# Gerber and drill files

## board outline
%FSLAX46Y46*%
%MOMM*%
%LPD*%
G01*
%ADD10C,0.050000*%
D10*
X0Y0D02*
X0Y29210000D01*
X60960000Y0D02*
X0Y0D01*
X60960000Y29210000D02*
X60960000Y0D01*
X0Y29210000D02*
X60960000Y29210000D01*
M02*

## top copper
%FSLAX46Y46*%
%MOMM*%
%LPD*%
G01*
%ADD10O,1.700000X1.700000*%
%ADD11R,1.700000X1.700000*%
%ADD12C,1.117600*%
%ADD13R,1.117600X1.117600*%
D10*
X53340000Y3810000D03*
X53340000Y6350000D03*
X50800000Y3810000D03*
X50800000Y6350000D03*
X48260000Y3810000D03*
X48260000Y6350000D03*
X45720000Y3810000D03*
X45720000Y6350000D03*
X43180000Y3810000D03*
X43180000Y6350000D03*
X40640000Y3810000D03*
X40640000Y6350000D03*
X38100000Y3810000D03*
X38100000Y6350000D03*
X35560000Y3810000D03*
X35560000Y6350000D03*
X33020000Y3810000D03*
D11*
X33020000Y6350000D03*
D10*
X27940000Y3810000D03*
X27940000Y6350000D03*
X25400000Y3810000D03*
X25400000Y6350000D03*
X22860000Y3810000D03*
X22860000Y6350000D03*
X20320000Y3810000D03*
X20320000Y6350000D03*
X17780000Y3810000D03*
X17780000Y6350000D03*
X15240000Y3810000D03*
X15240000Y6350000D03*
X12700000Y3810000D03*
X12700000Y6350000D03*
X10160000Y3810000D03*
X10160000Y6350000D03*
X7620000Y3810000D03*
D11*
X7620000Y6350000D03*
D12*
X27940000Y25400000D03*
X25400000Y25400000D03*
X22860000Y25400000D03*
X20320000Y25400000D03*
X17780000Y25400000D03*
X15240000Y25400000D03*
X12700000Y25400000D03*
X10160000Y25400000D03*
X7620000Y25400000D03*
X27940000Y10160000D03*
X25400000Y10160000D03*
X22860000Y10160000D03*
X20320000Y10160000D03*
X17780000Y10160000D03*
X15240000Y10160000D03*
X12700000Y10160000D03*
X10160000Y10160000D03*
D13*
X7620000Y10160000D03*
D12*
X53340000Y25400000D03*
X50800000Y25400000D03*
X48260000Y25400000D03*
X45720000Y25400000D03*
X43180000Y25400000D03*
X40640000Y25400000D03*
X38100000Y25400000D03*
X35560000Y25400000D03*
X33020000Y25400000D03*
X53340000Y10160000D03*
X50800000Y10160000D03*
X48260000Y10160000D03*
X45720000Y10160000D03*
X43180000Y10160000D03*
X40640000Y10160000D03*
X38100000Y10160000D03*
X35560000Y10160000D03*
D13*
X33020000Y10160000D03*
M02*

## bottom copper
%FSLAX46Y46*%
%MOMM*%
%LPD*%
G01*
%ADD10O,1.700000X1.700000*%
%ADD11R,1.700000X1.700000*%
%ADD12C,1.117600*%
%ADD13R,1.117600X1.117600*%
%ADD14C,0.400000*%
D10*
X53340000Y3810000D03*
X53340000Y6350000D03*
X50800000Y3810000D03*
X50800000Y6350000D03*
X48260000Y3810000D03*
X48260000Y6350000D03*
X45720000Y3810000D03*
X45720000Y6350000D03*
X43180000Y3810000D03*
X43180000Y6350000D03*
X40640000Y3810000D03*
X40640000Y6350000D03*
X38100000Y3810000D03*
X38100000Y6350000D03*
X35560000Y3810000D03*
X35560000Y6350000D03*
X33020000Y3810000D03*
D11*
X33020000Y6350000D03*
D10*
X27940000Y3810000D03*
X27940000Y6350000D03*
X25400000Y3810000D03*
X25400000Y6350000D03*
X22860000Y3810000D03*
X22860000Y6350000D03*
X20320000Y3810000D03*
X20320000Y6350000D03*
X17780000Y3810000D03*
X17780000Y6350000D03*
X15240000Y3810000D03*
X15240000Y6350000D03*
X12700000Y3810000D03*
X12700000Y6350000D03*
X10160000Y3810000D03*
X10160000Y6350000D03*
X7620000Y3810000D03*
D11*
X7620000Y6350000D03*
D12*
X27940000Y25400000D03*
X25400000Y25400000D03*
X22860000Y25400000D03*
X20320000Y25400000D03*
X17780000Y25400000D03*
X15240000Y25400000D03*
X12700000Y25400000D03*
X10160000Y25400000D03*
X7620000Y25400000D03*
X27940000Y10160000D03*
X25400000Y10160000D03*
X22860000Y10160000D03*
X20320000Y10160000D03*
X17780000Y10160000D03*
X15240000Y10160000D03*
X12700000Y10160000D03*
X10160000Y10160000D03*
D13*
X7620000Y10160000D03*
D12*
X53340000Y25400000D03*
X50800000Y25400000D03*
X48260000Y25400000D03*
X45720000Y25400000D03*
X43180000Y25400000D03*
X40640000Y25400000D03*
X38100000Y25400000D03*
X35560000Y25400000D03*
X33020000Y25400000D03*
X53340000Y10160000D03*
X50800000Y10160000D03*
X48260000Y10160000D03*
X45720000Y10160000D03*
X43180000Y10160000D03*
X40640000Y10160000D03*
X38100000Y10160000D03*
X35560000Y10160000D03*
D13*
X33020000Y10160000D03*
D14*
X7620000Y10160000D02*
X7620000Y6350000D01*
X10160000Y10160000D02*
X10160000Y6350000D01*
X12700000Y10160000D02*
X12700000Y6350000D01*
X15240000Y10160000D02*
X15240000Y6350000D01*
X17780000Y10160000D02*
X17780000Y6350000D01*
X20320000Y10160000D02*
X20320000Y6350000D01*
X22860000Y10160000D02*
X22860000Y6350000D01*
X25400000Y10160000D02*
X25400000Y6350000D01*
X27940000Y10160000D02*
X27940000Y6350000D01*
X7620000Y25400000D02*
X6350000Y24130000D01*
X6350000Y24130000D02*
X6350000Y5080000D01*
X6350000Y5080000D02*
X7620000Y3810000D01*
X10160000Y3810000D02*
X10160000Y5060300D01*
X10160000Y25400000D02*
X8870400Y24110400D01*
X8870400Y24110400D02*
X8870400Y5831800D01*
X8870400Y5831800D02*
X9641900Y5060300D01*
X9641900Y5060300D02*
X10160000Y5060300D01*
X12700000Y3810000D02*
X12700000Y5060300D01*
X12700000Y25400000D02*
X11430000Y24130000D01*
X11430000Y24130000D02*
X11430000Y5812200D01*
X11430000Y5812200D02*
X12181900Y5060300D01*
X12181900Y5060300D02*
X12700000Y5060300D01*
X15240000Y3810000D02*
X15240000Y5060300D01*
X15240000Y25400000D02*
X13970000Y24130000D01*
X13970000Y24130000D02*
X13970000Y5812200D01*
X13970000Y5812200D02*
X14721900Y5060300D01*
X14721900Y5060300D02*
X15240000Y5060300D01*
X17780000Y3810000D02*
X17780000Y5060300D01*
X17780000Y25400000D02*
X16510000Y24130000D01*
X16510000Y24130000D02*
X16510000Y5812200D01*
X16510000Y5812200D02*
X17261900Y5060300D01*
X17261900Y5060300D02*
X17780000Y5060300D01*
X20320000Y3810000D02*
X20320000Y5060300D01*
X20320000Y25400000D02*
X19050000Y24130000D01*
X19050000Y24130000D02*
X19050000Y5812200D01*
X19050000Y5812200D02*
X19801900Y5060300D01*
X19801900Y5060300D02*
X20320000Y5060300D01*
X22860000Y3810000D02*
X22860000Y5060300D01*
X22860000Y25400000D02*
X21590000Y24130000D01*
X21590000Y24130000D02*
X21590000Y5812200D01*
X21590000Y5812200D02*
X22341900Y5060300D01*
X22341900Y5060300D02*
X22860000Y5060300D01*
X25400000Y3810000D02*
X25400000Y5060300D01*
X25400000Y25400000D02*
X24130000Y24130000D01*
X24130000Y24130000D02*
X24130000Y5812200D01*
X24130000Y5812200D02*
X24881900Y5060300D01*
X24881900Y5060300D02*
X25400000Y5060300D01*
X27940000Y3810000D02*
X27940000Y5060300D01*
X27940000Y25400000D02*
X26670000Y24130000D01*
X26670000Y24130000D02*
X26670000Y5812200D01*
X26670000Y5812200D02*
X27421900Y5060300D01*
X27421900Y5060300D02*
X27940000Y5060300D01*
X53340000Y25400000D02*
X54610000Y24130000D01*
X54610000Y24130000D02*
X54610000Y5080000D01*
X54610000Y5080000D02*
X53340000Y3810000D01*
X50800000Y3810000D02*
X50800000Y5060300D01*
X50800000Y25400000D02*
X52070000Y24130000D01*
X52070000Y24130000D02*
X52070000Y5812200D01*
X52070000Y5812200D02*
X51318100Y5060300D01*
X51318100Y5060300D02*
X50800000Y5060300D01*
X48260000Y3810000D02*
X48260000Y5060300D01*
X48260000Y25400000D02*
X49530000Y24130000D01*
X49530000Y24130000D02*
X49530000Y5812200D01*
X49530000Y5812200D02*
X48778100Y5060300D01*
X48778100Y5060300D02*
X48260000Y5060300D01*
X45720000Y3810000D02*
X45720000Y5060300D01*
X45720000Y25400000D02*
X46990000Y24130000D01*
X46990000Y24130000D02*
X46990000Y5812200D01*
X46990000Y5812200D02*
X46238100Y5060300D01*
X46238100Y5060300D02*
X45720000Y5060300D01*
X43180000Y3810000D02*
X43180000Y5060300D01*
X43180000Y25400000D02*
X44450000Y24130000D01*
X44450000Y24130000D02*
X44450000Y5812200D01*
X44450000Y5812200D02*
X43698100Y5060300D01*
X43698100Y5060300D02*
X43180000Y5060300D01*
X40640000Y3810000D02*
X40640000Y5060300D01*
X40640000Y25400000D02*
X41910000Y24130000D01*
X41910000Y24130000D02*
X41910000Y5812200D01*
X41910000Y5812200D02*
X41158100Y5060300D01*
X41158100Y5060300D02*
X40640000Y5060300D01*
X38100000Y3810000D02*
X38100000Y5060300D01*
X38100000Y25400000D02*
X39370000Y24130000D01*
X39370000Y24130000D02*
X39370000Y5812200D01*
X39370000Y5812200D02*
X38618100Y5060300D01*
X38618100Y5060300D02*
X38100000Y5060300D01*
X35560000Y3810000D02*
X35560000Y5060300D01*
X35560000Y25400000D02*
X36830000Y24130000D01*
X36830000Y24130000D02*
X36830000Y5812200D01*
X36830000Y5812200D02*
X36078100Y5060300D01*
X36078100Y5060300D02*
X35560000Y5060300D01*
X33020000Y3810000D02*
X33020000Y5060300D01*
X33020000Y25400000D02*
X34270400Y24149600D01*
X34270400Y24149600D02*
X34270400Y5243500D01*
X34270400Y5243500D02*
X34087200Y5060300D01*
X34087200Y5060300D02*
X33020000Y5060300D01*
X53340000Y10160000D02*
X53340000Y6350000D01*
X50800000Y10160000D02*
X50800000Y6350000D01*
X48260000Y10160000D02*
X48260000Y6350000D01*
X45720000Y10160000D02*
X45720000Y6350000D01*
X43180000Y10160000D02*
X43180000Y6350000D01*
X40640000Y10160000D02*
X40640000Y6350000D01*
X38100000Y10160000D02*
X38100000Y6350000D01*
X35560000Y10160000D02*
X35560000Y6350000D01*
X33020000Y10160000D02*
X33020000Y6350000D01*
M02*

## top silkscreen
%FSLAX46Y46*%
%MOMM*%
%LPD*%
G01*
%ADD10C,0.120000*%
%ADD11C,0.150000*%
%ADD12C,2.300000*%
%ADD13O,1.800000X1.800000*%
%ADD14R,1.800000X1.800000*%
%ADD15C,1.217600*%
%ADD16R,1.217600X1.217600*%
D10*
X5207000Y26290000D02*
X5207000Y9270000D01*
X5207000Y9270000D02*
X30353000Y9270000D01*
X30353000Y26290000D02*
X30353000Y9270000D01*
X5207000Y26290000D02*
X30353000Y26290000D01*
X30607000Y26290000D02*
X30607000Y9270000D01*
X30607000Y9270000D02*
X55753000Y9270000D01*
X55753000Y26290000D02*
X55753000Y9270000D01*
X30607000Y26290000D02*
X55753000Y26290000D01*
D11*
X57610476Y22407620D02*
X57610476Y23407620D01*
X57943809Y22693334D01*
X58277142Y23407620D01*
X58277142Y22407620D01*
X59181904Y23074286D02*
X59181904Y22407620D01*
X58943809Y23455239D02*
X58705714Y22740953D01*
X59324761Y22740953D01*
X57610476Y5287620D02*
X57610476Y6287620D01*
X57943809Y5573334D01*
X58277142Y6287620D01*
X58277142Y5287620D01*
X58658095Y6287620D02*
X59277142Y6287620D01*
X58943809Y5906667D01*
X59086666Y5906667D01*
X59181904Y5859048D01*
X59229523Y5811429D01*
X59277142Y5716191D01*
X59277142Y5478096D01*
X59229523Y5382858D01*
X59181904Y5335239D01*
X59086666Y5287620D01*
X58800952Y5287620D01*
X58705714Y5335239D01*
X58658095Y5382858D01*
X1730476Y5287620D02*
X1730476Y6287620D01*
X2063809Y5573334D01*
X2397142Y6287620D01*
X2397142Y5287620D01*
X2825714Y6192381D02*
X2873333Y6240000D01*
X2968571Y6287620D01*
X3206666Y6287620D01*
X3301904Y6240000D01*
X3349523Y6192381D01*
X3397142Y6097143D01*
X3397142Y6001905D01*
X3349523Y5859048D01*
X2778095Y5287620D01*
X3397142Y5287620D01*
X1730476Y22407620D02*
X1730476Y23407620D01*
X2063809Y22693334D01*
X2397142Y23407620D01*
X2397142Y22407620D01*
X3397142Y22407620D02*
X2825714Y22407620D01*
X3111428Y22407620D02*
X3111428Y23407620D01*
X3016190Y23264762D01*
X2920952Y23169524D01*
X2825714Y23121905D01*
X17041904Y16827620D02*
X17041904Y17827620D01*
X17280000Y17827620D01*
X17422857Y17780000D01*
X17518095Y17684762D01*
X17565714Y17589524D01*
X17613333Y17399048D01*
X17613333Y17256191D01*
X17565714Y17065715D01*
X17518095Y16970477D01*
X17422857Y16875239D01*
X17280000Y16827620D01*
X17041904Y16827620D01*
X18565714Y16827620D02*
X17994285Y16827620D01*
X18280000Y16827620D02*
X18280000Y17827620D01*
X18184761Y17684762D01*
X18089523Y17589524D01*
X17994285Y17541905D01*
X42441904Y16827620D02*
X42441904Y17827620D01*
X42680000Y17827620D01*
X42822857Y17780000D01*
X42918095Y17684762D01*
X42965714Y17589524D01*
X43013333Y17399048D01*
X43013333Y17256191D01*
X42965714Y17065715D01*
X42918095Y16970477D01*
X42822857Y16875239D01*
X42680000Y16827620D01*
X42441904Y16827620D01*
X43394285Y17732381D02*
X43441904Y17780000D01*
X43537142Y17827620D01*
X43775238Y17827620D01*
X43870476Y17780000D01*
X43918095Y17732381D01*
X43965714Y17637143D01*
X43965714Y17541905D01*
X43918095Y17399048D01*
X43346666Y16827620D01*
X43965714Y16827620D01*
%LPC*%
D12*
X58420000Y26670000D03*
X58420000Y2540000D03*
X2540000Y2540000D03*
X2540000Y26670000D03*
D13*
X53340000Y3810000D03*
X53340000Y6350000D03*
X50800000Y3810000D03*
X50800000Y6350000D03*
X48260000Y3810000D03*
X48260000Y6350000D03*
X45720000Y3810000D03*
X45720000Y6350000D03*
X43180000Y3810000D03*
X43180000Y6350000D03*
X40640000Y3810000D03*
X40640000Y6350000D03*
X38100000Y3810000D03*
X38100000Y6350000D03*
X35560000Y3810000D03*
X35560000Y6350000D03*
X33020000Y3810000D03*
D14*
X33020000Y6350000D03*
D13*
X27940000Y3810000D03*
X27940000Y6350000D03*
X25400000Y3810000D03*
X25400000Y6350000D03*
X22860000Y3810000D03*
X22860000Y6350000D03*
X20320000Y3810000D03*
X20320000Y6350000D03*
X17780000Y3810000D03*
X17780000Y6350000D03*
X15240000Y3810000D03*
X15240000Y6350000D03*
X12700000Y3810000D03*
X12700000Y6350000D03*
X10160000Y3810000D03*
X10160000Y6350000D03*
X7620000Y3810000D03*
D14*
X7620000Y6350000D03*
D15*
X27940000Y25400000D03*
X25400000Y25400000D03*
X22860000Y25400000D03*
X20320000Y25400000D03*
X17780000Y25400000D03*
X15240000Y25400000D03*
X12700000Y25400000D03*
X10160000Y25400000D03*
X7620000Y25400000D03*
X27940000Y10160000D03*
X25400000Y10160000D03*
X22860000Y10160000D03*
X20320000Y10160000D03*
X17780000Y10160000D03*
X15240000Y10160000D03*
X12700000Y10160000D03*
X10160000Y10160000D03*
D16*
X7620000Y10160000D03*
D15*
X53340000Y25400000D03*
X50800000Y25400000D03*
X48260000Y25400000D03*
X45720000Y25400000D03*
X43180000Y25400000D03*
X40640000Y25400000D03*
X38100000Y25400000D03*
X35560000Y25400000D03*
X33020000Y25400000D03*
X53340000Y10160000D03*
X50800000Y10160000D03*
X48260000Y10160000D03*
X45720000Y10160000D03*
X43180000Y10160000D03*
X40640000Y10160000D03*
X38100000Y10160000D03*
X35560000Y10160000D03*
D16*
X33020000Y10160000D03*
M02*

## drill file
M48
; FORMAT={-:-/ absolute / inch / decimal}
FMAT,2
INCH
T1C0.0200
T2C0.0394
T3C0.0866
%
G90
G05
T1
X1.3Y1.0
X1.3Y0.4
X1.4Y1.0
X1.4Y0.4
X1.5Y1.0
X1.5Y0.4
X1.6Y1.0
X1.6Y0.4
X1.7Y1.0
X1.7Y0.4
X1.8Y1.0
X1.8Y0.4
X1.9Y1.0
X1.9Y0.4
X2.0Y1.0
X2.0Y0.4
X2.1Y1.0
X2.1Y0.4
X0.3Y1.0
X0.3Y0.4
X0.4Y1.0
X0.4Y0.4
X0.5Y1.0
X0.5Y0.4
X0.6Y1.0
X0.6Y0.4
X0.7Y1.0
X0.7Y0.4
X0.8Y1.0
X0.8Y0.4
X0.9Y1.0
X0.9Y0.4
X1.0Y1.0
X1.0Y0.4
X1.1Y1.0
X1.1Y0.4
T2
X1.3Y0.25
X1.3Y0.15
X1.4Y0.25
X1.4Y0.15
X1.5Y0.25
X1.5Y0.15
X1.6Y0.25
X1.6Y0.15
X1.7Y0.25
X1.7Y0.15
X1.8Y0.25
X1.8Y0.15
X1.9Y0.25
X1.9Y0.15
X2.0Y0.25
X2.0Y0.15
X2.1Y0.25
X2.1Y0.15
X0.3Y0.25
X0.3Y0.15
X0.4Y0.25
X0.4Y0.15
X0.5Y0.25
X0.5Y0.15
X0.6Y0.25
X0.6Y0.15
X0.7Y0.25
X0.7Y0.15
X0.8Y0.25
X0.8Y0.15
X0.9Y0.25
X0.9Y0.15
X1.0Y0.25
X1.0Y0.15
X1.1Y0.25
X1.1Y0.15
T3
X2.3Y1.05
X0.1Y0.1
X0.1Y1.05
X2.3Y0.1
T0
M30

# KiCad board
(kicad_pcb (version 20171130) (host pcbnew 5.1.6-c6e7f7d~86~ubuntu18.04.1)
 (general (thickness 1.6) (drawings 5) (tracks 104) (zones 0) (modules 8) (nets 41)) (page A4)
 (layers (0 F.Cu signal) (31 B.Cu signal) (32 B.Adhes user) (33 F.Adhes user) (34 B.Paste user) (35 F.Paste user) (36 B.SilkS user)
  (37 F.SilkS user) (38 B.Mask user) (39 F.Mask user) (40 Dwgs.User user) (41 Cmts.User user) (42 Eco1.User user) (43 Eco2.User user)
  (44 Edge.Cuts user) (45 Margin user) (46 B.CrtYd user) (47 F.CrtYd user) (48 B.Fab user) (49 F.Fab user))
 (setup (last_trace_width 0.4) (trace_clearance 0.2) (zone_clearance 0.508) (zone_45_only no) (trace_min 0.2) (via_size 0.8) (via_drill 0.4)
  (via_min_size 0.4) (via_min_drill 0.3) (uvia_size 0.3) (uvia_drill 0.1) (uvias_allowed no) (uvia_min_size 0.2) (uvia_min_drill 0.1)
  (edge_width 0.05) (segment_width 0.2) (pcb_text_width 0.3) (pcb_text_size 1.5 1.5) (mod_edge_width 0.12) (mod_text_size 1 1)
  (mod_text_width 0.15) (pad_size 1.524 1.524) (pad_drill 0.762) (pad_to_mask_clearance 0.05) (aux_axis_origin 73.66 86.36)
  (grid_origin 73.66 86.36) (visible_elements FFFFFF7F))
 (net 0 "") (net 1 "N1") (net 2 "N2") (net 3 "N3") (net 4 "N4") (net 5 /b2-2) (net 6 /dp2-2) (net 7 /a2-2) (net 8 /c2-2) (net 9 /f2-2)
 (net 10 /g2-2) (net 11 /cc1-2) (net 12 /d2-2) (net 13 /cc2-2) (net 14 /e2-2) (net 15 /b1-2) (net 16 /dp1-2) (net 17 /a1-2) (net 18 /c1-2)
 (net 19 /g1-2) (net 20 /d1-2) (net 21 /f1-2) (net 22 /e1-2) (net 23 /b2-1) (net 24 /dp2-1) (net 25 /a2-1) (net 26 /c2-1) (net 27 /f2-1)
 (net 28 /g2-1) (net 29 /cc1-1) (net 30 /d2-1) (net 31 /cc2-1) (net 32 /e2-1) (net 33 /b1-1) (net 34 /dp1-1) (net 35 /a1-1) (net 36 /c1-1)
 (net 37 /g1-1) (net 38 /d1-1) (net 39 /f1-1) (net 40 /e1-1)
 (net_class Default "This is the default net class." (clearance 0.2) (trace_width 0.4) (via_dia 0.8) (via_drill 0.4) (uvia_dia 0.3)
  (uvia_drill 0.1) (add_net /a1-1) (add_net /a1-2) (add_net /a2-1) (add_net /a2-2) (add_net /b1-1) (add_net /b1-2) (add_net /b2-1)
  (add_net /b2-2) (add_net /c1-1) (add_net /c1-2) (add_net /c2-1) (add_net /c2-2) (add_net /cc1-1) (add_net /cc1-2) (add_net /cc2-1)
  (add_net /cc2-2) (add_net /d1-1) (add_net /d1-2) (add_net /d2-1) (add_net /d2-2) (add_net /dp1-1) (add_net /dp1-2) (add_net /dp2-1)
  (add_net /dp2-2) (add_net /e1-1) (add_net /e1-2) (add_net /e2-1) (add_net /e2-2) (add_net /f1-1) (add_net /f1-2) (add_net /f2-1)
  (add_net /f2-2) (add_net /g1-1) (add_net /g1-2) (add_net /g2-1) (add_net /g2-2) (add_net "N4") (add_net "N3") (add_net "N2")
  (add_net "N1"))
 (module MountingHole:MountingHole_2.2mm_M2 (layer F.Cu) (at 132.08 59.69)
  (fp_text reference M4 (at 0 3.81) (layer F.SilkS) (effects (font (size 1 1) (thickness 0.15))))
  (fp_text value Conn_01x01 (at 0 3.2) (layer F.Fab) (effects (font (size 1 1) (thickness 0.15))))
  (pad 1 np_thru_hole circle (at 0 0) (size 2.2 2.2) (drill 2.2) (layers *.Cu *.Mask) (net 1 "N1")))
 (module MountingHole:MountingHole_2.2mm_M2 (layer F.Cu) (at 132.08 83.82)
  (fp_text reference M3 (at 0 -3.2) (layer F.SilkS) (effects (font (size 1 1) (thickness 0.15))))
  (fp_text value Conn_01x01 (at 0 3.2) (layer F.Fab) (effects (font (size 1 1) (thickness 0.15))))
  (pad 1 np_thru_hole circle (at 0 0) (size 2.2 2.2) (drill 2.2) (layers *.Cu *.Mask) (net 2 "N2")))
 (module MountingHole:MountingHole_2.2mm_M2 (layer F.Cu) (at 76.2 83.82)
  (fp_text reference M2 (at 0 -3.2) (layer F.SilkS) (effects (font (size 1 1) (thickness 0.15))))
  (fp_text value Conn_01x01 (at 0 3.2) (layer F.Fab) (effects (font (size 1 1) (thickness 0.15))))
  (pad 1 np_thru_hole circle (at 0 0) (size 2.2 2.2) (drill 2.2) (layers *.Cu *.Mask) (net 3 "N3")))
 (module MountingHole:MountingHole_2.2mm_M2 (layer F.Cu) (at 76.2 59.69)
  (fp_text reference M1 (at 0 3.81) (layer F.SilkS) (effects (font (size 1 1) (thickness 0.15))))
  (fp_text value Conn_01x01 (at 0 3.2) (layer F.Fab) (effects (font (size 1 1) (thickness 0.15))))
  (pad 1 np_thru_hole circle (at 0 0) (size 2.2 2.2) (drill 2.2) (layers *.Cu *.Mask) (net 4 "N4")))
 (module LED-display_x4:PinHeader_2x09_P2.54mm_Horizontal (layer B.Cu) (at 106.68 80.01 270)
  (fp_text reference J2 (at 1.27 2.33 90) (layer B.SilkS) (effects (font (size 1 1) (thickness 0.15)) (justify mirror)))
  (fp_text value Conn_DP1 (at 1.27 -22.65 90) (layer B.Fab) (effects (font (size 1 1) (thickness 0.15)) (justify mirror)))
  (pad 10 thru_hole oval (at 2.54 -20.32 270) (size 1.7 1.7) (drill 1) (layers *.Cu *.Mask) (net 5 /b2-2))
  (pad 9 thru_hole oval (at 0 -20.32 270) (size 1.7 1.7) (drill 1) (layers *.Cu *.Mask) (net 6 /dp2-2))
  (pad 11 thru_hole oval (at 2.54 -17.78 270) (size 1.7 1.7) (drill 1) (layers *.Cu *.Mask) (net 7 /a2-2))
  (pad 8 thru_hole oval (at 0 -17.78 270) (size 1.7 1.7) (drill 1) (layers *.Cu *.Mask) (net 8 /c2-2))
  (pad 12 thru_hole oval (at 2.54 -15.24 270) (size 1.7 1.7) (drill 1) (layers *.Cu *.Mask) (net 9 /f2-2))
  (pad 7 thru_hole oval (at 0 -15.24 270) (size 1.7 1.7) (drill 1) (layers *.Cu *.Mask) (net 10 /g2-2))
  (pad 13 thru_hole oval (at 2.54 -12.7 270) (size 1.7 1.7) (drill 1) (layers *.Cu *.Mask) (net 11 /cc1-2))
  (pad 6 thru_hole oval (at 0 -12.7 270) (size 1.7 1.7) (drill 1) (layers *.Cu *.Mask) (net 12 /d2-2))
  (pad 14 thru_hole oval (at 2.54 -10.16 270) (size 1.7 1.7) (drill 1) (layers *.Cu *.Mask) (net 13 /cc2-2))
  (pad 5 thru_hole oval (at 0 -10.16 270) (size 1.7 1.7) (drill 1) (layers *.Cu *.Mask) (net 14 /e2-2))
  (pad 15 thru_hole oval (at 2.54 -7.62 270) (size 1.7 1.7) (drill 1) (layers *.Cu *.Mask) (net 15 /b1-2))
  (pad 4 thru_hole oval (at 0 -7.62 270) (size 1.7 1.7) (drill 1) (layers *.Cu *.Mask) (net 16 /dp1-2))
  (pad 16 thru_hole oval (at 2.54 -5.08 270) (size 1.7 1.7) (drill 1) (layers *.Cu *.Mask) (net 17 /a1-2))
  (pad 3 thru_hole oval (at 0 -5.08 270) (size 1.7 1.7) (drill 1) (layers *.Cu *.Mask) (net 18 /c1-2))
  (pad 17 thru_hole oval (at 2.54 -2.54 270) (size 1.7 1.7) (drill 1) (layers *.Cu *.Mask) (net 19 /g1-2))
  (pad 2 thru_hole oval (at 0 -2.54 270) (size 1.7 1.7) (drill 1) (layers *.Cu *.Mask) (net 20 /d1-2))
  (pad 18 thru_hole oval (at 2.54 0 270) (size 1.7 1.7) (drill 1) (layers *.Cu *.Mask) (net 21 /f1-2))
  (pad 1 thru_hole rect (at 0 0 270) (size 1.7 1.7) (drill 1) (layers *.Cu *.Mask) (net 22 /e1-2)))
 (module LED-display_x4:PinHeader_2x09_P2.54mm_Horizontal (layer B.Cu) (at 81.28 80.01 270)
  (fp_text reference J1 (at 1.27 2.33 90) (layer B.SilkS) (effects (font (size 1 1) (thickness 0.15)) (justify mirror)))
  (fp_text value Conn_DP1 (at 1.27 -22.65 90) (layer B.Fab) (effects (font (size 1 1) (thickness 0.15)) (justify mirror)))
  (pad 10 thru_hole oval (at 2.54 -20.32 270) (size 1.7 1.7) (drill 1) (layers *.Cu *.Mask) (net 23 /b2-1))
  (pad 9 thru_hole oval (at 0 -20.32 270) (size 1.7 1.7) (drill 1) (layers *.Cu *.Mask) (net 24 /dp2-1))
  (pad 11 thru_hole oval (at 2.54 -17.78 270) (size 1.7 1.7) (drill 1) (layers *.Cu *.Mask) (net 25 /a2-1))
  (pad 8 thru_hole oval (at 0 -17.78 270) (size 1.7 1.7) (drill 1) (layers *.Cu *.Mask) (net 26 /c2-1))
  (pad 12 thru_hole oval (at 2.54 -15.24 270) (size 1.7 1.7) (drill 1) (layers *.Cu *.Mask) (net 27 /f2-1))
  (pad 7 thru_hole oval (at 0 -15.24 270) (size 1.7 1.7) (drill 1) (layers *.Cu *.Mask) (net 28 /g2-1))
  (pad 13 thru_hole oval (at 2.54 -12.7 270) (size 1.7 1.7) (drill 1) (layers *.Cu *.Mask) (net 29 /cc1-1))
  (pad 6 thru_hole oval (at 0 -12.7 270) (size 1.7 1.7) (drill 1) (layers *.Cu *.Mask) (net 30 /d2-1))
  (pad 14 thru_hole oval (at 2.54 -10.16 270) (size 1.7 1.7) (drill 1) (layers *.Cu *.Mask) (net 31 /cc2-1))
  (pad 5 thru_hole oval (at 0 -10.16 270) (size 1.7 1.7) (drill 1) (layers *.Cu *.Mask) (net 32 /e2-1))
  (pad 15 thru_hole oval (at 2.54 -7.62 270) (size 1.7 1.7) (drill 1) (layers *.Cu *.Mask) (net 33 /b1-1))
  (pad 4 thru_hole oval (at 0 -7.62 270) (size 1.7 1.7) (drill 1) (layers *.Cu *.Mask) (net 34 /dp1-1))
  (pad 16 thru_hole oval (at 2.54 -5.08 270) (size 1.7 1.7) (drill 1) (layers *.Cu *.Mask) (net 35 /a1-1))
  (pad 3 thru_hole oval (at 0 -5.08 270) (size 1.7 1.7) (drill 1) (layers *.Cu *.Mask) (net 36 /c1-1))
  (pad 17 thru_hole oval (at 2.54 -2.54 270) (size 1.7 1.7) (drill 1) (layers *.Cu *.Mask) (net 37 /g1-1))
  (pad 2 thru_hole oval (at 0 -2.54 270) (size 1.7 1.7) (drill 1) (layers *.Cu *.Mask) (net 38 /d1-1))
  (pad 18 thru_hole oval (at 2.54 0 270) (size 1.7 1.7) (drill 1) (layers *.Cu *.Mask) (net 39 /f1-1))
  (pad 1 thru_hole rect (at 0 0 270) (size 1.7 1.7) (drill 1) (layers *.Cu *.Mask) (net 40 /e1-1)))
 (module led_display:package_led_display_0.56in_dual (layer F.Cu) (at 91.44 68.58)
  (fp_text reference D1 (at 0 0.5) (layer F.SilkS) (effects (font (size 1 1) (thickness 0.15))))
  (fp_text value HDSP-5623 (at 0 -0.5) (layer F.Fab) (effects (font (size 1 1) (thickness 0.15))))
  (fp_line (start -12.573 -8.51) (end -12.573 8.51) (layer F.SilkS) (width 0.12))
  (fp_line (start -12.573 8.51) (end 12.573 8.51) (layer F.SilkS) (width 0.12))
  (fp_line (start 12.573 -8.51) (end 12.573 8.51) (layer F.SilkS) (width 0.12))
  (fp_line (start -12.573 -8.51) (end 12.573 -8.51) (layer F.SilkS) (width 0.12))
  (pad 10 thru_hole circle (at 10.16 -7.62) (size 1.1176 1.1176) (drill 0.508) (layers *.Cu *.Mask) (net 23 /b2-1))
  (pad 11 thru_hole circle (at 7.62 -7.62) (size 1.1176 1.1176) (drill 0.508) (layers *.Cu *.Mask) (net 25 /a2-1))
  (pad 12 thru_hole circle (at 5.08 -7.62) (size 1.1176 1.1176) (drill 0.508) (layers *.Cu *.Mask) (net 27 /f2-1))
  (pad 13 thru_hole circle (at 2.54 -7.62) (size 1.1176 1.1176) (drill 0.508) (layers *.Cu *.Mask) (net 29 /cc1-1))
  (pad 14 thru_hole circle (at 0 -7.62) (size 1.1176 1.1176) (drill 0.508) (layers *.Cu *.Mask) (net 31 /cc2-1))
  (pad 15 thru_hole circle (at -2.54 -7.62) (size 1.1176 1.1176) (drill 0.508) (layers *.Cu *.Mask) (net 33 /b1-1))
  (pad 16 thru_hole circle (at -5.08 -7.62) (size 1.1176 1.1176) (drill 0.508) (layers *.Cu *.Mask) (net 35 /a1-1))
  (pad 17 thru_hole circle (at -7.62 -7.62) (size 1.1176 1.1176) (drill 0.508) (layers *.Cu *.Mask) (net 37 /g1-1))
  (pad 18 thru_hole circle (at -10.16 -7.62) (size 1.1176 1.1176) (drill 0.508) (layers *.Cu *.Mask) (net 39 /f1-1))
  (pad 9 thru_hole circle (at 10.16 7.62) (size 1.1176 1.1176) (drill 0.508) (layers *.Cu *.Mask) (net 24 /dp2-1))
  (pad 8 thru_hole circle (at 7.62 7.62) (size 1.1176 1.1176) (drill 0.508) (layers *.Cu *.Mask) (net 26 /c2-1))
  (pad 7 thru_hole circle (at 5.08 7.62) (size 1.1176 1.1176) (drill 0.508) (layers *.Cu *.Mask) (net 28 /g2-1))
  (pad 6 thru_hole circle (at 2.54 7.62) (size 1.1176 1.1176) (drill 0.508) (layers *.Cu *.Mask) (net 30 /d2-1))
  (pad 5 thru_hole circle (at 0 7.62) (size 1.1176 1.1176) (drill 0.508) (layers *.Cu *.Mask) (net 32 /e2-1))
  (pad 4 thru_hole circle (at -2.54 7.62) (size 1.1176 1.1176) (drill 0.508) (layers *.Cu *.Mask) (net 34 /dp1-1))
  (pad 3 thru_hole circle (at -5.08 7.62) (size 1.1176 1.1176) (drill 0.508) (layers *.Cu *.Mask) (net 36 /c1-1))
  (pad 2 thru_hole circle (at -7.62 7.62) (size 1.1176 1.1176) (drill 0.508) (layers *.Cu *.Mask) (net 38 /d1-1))
  (pad 1 thru_hole rect (at -10.16 7.62) (size 1.1176 1.1176) (drill 0.508) (layers *.Cu *.Mask) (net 40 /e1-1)))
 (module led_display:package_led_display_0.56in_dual (layer F.Cu) (at 116.84 68.58)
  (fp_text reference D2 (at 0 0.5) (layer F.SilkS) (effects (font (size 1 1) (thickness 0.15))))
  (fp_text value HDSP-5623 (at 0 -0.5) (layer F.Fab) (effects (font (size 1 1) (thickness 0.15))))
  (fp_line (start -12.573 -8.51) (end -12.573 8.51) (layer F.SilkS) (width 0.12))
  (fp_line (start -12.573 8.51) (end 12.573 8.51) (layer F.SilkS) (width 0.12))
  (fp_line (start 12.573 -8.51) (end 12.573 8.51) (layer F.SilkS) (width 0.12))
  (fp_line (start -12.573 -8.51) (end 12.573 -8.51) (layer F.SilkS) (width 0.12))
  (pad 10 thru_hole circle (at 10.16 -7.62) (size 1.1176 1.1176) (drill 0.508) (layers *.Cu *.Mask) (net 5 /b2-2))
  (pad 11 thru_hole circle (at 7.62 -7.62) (size 1.1176 1.1176) (drill 0.508) (layers *.Cu *.Mask) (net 7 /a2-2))
  (pad 12 thru_hole circle (at 5.08 -7.62) (size 1.1176 1.1176) (drill 0.508) (layers *.Cu *.Mask) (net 9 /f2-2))
  (pad 13 thru_hole circle (at 2.54 -7.62) (size 1.1176 1.1176) (drill 0.508) (layers *.Cu *.Mask) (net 11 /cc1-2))
  (pad 14 thru_hole circle (at 0 -7.62) (size 1.1176 1.1176) (drill 0.508) (layers *.Cu *.Mask) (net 13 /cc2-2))
  (pad 15 thru_hole circle (at -2.54 -7.62) (size 1.1176 1.1176) (drill 0.508) (layers *.Cu *.Mask) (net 15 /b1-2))
  (pad 16 thru_hole circle (at -5.08 -7.62) (size 1.1176 1.1176) (drill 0.508) (layers *.Cu *.Mask) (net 17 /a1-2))
  (pad 17 thru_hole circle (at -7.62 -7.62) (size 1.1176 1.1176) (drill 0.508) (layers *.Cu *.Mask) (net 19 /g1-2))
  (pad 18 thru_hole circle (at -10.16 -7.62) (size 1.1176 1.1176) (drill 0.508) (layers *.Cu *.Mask) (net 21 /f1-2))
  (pad 9 thru_hole circle (at 10.16 7.62) (size 1.1176 1.1176) (drill 0.508) (layers *.Cu *.Mask) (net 6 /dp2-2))
  (pad 8 thru_hole circle (at 7.62 7.62) (size 1.1176 1.1176) (drill 0.508) (layers *.Cu *.Mask) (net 8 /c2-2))
  (pad 7 thru_hole circle (at 5.08 7.62) (size 1.1176 1.1176) (drill 0.508) (layers *.Cu *.Mask) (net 10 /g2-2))
  (pad 6 thru_hole circle (at 2.54 7.62) (size 1.1176 1.1176) (drill 0.508) (layers *.Cu *.Mask) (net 12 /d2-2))
  (pad 5 thru_hole circle (at 0 7.62) (size 1.1176 1.1176) (drill 0.508) (layers *.Cu *.Mask) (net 14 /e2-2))
  (pad 4 thru_hole circle (at -2.54 7.62) (size 1.1176 1.1176) (drill 0.508) (layers *.Cu *.Mask) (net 16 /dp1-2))
  (pad 3 thru_hole circle (at -5.08 7.62) (size 1.1176 1.1176) (drill 0.508) (layers *.Cu *.Mask) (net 18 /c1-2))
  (pad 2 thru_hole circle (at -7.62 7.62) (size 1.1176 1.1176) (drill 0.508) (layers *.Cu *.Mask) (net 20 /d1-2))
  (pad 1 thru_hole rect (at -10.16 7.62) (size 1.1176 1.1176) (drill 0.508) (layers *.Cu *.Mask) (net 22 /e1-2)))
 (gr_line (start 73.66 86.36) (end 73.66 57.15) (layer Edge.Cuts) (width 0.05))
 (gr_line (start 134.62 86.36) (end 73.66 86.36) (layer Edge.Cuts) (width 0.05))
 (gr_line (start 134.62 57.15) (end 134.62 86.36) (layer Edge.Cuts) (width 0.05))
 (gr_line (start 73.66 57.15) (end 134.62 57.15) (layer Edge.Cuts) (width 0.05))
 (segment (start 81.28 76.2) (end 81.28 80.01) (width 0.4) (layer B.Cu) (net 40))
 (segment (start 83.82 76.2) (end 83.82 80.01) (width 0.4) (layer B.Cu) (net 38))
 (segment (start 86.36 76.2) (end 86.36 80.01) (width 0.4) (layer B.Cu) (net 36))
 (segment (start 88.9 76.2) (end 88.9 80.01) (width 0.4) (layer B.Cu) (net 34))
 (segment (start 91.44 76.2) (end 91.44 80.01) (width 0.4) (layer B.Cu) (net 32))
 (segment (start 93.98 76.2) (end 93.98 80.01) (width 0.4) (layer B.Cu) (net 30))
 (segment (start 96.52 76.2) (end 96.52 80.01) (width 0.4) (layer B.Cu) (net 28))
 (segment (start 99.06 76.2) (end 99.06 80.01) (width 0.4) (layer B.Cu) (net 26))
 (segment (start 101.6 76.2) (end 101.6 80.01) (width 0.4) (layer B.Cu) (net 24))
 (segment (start 81.28 60.96) (end 80.01 62.23) (width 0.4) (layer B.Cu) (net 39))
 (segment (start 80.01 62.23) (end 80.01 81.28) (width 0.4) (layer B.Cu) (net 39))
 (segment (start 80.01 81.28) (end 81.28 82.55) (width 0.4) (layer B.Cu) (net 39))
 (segment (start 83.82 82.55) (end 83.82 81.2997) (width 0.4) (layer B.Cu) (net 37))
 (segment (start 83.82 60.96) (end 82.5304 62.2496) (width 0.4) (layer B.Cu) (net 37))
 (segment (start 82.5304 62.2496) (end 82.5304 80.5282) (width 0.4) (layer B.Cu) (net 37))
 (segment (start 82.5304 80.5282) (end 83.3019 81.2997) (width 0.4) (layer B.Cu) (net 37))
 (segment (start 83.3019 81.2997) (end 83.82 81.2997) (width 0.4) (layer B.Cu) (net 37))
 (segment (start 86.36 82.55) (end 86.36 81.2997) (width 0.4) (layer B.Cu) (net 35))
 (segment (start 86.36 60.96) (end 85.09 62.23) (width 0.4) (layer B.Cu) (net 35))
 (segment (start 85.09 62.23) (end 85.09 80.5478) (width 0.4) (layer B.Cu) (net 35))
 (segment (start 85.09 80.5478) (end 85.8419 81.2997) (width 0.4) (layer B.Cu) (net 35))
 (segment (start 85.8419 81.2997) (end 86.36 81.2997) (width 0.4) (layer B.Cu) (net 35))
 (segment (start 88.9 82.55) (end 88.9 81.2997) (width 0.4) (layer B.Cu) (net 33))
 (segment (start 88.9 60.96) (end 87.63 62.23) (width 0.4) (layer B.Cu) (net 33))
 (segment (start 87.63 62.23) (end 87.63 80.5478) (width 0.4) (layer B.Cu) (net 33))
 (segment (start 87.63 80.5478) (end 88.3819 81.2997) (width 0.4) (layer B.Cu) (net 33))
 (segment (start 88.3819 81.2997) (end 88.9 81.2997) (width 0.4) (layer B.Cu) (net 33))
 (segment (start 91.44 82.55) (end 91.44 81.2997) (width 0.4) (layer B.Cu) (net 31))
 (segment (start 91.44 60.96) (end 90.17 62.23) (width 0.4) (layer B.Cu) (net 31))
 (segment (start 90.17 62.23) (end 90.17 80.5478) (width 0.4) (layer B.Cu) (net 31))
 (segment (start 90.17 80.5478) (end 90.9219 81.2997) (width 0.4) (layer B.Cu) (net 31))
 (segment (start 90.9219 81.2997) (end 91.44 81.2997) (width 0.4) (layer B.Cu) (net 31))
 (segment (start 93.98 82.55) (end 93.98 81.2997) (width 0.4) (layer B.Cu) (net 29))
 (segment (start 93.98 60.96) (end 92.71 62.23) (width 0.4) (layer B.Cu) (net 29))
 (segment (start 92.71 62.23) (end 92.71 80.5478) (width 0.4) (layer B.Cu) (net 29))
 (segment (start 92.71 80.5478) (end 93.4619 81.2997) (width 0.4) (layer B.Cu) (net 29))
 (segment (start 93.4619 81.2997) (end 93.98 81.2997) (width 0.4) (layer B.Cu) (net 29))
 (segment (start 96.52 82.55) (end 96.52 81.2997) (width 0.4) (layer B.Cu) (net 27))
 (segment (start 96.52 60.96) (end 95.25 62.23) (width 0.4) (layer B.Cu) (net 27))
 (segment (start 95.25 62.23) (end 95.25 80.5478) (width 0.4) (layer B.Cu) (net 27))
 (segment (start 95.25 80.5478) (end 96.0019 81.2997) (width 0.4) (layer B.Cu) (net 27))
 (segment (start 96.0019 81.2997) (end 96.52 81.2997) (width 0.4) (layer B.Cu) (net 27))
 (segment (start 99.06 82.55) (end 99.06 81.2997) (width 0.4) (layer B.Cu) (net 25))
 (segment (start 99.06 60.96) (end 97.79 62.23) (width 0.4) (layer B.Cu) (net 25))
 (segment (start 97.79 62.23) (end 97.79 80.5478) (width 0.4) (layer B.Cu) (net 25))
 (segment (start 97.79 80.5478) (end 98.5419 81.2997) (width 0.4) (layer B.Cu) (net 25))
 (segment (start 98.5419 81.2997) (end 99.06 81.2997) (width 0.4) (layer B.Cu) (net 25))
 (segment (start 101.6 82.55) (end 101.6 81.2997) (width 0.4) (layer B.Cu) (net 23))
 (segment (start 101.6 60.96) (end 100.33 62.23) (width 0.4) (layer B.Cu) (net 23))
 (segment (start 100.33 62.23) (end 100.33 80.5478) (width 0.4) (layer B.Cu) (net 23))
 (segment (start 100.33 80.5478) (end 101.0819 81.2997) (width 0.4) (layer B.Cu) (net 23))
 (segment (start 101.0819 81.2997) (end 101.6 81.2997) (width 0.4) (layer B.Cu) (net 23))
 (segment (start 127 60.96) (end 128.27 62.23) (width 0.4) (layer B.Cu) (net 5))
 (segment (start 128.27 62.23) (end 128.27 81.28) (width 0.4) (layer B.Cu) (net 5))
 (segment (start 128.27 81.28) (end 127 82.55) (width 0.4) (layer B.Cu) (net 5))
 (segment (start 124.46 82.55) (end 124.46 81.2997) (width 0.4) (layer B.Cu) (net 7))
 (segment (start 124.46 60.96) (end 125.73 62.23) (width 0.4) (layer B.Cu) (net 7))
 (segment (start 125.73 62.23) (end 125.73 80.5478) (width 0.4) (layer B.Cu) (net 7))
 (segment (start 125.73 80.5478) (end 124.9781 81.2997) (width 0.4) (layer B.Cu) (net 7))
 (segment (start 124.9781 81.2997) (end 124.46 81.2997) (width 0.4) (layer B.Cu) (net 7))
 (segment (start 121.92 82.55) (end 121.92 81.2997) (width 0.4) (layer B.Cu) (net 9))
 (segment (start 121.92 60.96) (end 123.19 62.23) (width 0.4) (layer B.Cu) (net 9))
 (segment (start 123.19 62.23) (end 123.19 80.5478) (width 0.4) (layer B.Cu) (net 9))
 (segment (start 123.19 80.5478) (end 122.4381 81.2997) (width 0.4) (layer B.Cu) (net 9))
 (segment (start 122.4381 81.2997) (end 121.92 81.2997) (width 0.4) (layer B.Cu) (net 9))
 (segment (start 119.38 82.55) (end 119.38 81.2997) (width 0.4) (layer B.Cu) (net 11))
 (segment (start 119.38 60.96) (end 120.65 62.23) (width 0.4) (layer B.Cu) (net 11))
 (segment (start 120.65 62.23) (end 120.65 80.5478) (width 0.4) (layer B.Cu) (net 11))
 (segment (start 120.65 80.5478) (end 119.8981 81.2997) (width 0.4) (layer B.Cu) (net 11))
 (segment (start 119.8981 81.2997) (end 119.38 81.2997) (width 0.4) (layer B.Cu) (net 11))
 (segment (start 116.84 82.55) (end 116.84 81.2997) (width 0.4) (layer B.Cu) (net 13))
 (segment (start 116.84 60.96) (end 118.11 62.23) (width 0.4) (layer B.Cu) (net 13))
 (segment (start 118.11 62.23) (end 118.11 80.5478) (width 0.4) (layer B.Cu) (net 13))
 (segment (start 118.11 80.5478) (end 117.3581 81.2997) (width 0.4) (layer B.Cu) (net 13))
 (segment (start 117.3581 81.2997) (end 116.84 81.2997) (width 0.4) (layer B.Cu) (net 13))
 (segment (start 114.3 82.55) (end 114.3 81.2997) (width 0.4) (layer B.Cu) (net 15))
 (segment (start 114.3 60.96) (end 115.57 62.23) (width 0.4) (layer B.Cu) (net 15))
 (segment (start 115.57 62.23) (end 115.57 80.5478) (width 0.4) (layer B.Cu) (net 15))
 (segment (start 115.57 80.5478) (end 114.8181 81.2997) (width 0.4) (layer B.Cu) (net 15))
 (segment (start 114.8181 81.2997) (end 114.3 81.2997) (width 0.4) (layer B.Cu) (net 15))
 (segment (start 111.76 82.55) (end 111.76 81.2997) (width 0.4) (layer B.Cu) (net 17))
 (segment (start 111.76 60.96) (end 113.03 62.23) (width 0.4) (layer B.Cu) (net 17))
 (segment (start 113.03 62.23) (end 113.03 80.5478) (width 0.4) (layer B.Cu) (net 17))
 (segment (start 113.03 80.5478) (end 112.2781 81.2997) (width 0.4) (layer B.Cu) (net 17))
 (segment (start 112.2781 81.2997) (end 111.76 81.2997) (width 0.4) (layer B.Cu) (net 17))
 (segment (start 109.22 82.55) (end 109.22 81.2997) (width 0.4) (layer B.Cu) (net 19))
 (segment (start 109.22 60.96) (end 110.49 62.23) (width 0.4) (layer B.Cu) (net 19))
 (segment (start 110.49 62.23) (end 110.49 80.5478) (width 0.4) (layer B.Cu) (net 19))
 (segment (start 110.49 80.5478) (end 109.7381 81.2997) (width 0.4) (layer B.Cu) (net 19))
 (segment (start 109.7381 81.2997) (end 109.22 81.2997) (width 0.4) (layer B.Cu) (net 19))
 (segment (start 106.68 82.55) (end 106.68 81.2997) (width 0.4) (layer B.Cu) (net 21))
 (segment (start 106.68 60.96) (end 107.9304 62.2104) (width 0.4) (layer B.Cu) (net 21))
 (segment (start 107.9304 62.2104) (end 107.9304 81.1165) (width 0.4) (layer B.Cu) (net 21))
 (segment (start 107.9304 81.1165) (end 107.7472 81.2997) (width 0.4) (layer B.Cu) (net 21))
 (segment (start 107.7472 81.2997) (end 106.68 81.2997) (width 0.4) (layer B.Cu) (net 21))
 (segment (start 127 76.2) (end 127 80.01) (width 0.4) (layer B.Cu) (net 6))
 (segment (start 124.46 76.2) (end 124.46 80.01) (width 0.4) (layer B.Cu) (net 8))
 (segment (start 121.92 76.2) (end 121.92 80.01) (width 0.4) (layer B.Cu) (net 10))
 (segment (start 119.38 76.2) (end 119.38 80.01) (width 0.4) (layer B.Cu) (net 12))
 (segment (start 116.84 76.2) (end 116.84 80.01) (width 0.4) (layer B.Cu) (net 14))
 (segment (start 114.3 76.2) (end 114.3 80.01) (width 0.4) (layer B.Cu) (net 16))
 (segment (start 111.76 76.2) (end 111.76 80.01) (width 0.4) (layer B.Cu) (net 18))
 (segment (start 109.22 76.2) (end 109.22 80.01) (width 0.4) (layer B.Cu) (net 20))
 (segment (start 106.68 76.2) (end 106.68 80.01) (width 0.4) (layer B.Cu) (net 22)))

